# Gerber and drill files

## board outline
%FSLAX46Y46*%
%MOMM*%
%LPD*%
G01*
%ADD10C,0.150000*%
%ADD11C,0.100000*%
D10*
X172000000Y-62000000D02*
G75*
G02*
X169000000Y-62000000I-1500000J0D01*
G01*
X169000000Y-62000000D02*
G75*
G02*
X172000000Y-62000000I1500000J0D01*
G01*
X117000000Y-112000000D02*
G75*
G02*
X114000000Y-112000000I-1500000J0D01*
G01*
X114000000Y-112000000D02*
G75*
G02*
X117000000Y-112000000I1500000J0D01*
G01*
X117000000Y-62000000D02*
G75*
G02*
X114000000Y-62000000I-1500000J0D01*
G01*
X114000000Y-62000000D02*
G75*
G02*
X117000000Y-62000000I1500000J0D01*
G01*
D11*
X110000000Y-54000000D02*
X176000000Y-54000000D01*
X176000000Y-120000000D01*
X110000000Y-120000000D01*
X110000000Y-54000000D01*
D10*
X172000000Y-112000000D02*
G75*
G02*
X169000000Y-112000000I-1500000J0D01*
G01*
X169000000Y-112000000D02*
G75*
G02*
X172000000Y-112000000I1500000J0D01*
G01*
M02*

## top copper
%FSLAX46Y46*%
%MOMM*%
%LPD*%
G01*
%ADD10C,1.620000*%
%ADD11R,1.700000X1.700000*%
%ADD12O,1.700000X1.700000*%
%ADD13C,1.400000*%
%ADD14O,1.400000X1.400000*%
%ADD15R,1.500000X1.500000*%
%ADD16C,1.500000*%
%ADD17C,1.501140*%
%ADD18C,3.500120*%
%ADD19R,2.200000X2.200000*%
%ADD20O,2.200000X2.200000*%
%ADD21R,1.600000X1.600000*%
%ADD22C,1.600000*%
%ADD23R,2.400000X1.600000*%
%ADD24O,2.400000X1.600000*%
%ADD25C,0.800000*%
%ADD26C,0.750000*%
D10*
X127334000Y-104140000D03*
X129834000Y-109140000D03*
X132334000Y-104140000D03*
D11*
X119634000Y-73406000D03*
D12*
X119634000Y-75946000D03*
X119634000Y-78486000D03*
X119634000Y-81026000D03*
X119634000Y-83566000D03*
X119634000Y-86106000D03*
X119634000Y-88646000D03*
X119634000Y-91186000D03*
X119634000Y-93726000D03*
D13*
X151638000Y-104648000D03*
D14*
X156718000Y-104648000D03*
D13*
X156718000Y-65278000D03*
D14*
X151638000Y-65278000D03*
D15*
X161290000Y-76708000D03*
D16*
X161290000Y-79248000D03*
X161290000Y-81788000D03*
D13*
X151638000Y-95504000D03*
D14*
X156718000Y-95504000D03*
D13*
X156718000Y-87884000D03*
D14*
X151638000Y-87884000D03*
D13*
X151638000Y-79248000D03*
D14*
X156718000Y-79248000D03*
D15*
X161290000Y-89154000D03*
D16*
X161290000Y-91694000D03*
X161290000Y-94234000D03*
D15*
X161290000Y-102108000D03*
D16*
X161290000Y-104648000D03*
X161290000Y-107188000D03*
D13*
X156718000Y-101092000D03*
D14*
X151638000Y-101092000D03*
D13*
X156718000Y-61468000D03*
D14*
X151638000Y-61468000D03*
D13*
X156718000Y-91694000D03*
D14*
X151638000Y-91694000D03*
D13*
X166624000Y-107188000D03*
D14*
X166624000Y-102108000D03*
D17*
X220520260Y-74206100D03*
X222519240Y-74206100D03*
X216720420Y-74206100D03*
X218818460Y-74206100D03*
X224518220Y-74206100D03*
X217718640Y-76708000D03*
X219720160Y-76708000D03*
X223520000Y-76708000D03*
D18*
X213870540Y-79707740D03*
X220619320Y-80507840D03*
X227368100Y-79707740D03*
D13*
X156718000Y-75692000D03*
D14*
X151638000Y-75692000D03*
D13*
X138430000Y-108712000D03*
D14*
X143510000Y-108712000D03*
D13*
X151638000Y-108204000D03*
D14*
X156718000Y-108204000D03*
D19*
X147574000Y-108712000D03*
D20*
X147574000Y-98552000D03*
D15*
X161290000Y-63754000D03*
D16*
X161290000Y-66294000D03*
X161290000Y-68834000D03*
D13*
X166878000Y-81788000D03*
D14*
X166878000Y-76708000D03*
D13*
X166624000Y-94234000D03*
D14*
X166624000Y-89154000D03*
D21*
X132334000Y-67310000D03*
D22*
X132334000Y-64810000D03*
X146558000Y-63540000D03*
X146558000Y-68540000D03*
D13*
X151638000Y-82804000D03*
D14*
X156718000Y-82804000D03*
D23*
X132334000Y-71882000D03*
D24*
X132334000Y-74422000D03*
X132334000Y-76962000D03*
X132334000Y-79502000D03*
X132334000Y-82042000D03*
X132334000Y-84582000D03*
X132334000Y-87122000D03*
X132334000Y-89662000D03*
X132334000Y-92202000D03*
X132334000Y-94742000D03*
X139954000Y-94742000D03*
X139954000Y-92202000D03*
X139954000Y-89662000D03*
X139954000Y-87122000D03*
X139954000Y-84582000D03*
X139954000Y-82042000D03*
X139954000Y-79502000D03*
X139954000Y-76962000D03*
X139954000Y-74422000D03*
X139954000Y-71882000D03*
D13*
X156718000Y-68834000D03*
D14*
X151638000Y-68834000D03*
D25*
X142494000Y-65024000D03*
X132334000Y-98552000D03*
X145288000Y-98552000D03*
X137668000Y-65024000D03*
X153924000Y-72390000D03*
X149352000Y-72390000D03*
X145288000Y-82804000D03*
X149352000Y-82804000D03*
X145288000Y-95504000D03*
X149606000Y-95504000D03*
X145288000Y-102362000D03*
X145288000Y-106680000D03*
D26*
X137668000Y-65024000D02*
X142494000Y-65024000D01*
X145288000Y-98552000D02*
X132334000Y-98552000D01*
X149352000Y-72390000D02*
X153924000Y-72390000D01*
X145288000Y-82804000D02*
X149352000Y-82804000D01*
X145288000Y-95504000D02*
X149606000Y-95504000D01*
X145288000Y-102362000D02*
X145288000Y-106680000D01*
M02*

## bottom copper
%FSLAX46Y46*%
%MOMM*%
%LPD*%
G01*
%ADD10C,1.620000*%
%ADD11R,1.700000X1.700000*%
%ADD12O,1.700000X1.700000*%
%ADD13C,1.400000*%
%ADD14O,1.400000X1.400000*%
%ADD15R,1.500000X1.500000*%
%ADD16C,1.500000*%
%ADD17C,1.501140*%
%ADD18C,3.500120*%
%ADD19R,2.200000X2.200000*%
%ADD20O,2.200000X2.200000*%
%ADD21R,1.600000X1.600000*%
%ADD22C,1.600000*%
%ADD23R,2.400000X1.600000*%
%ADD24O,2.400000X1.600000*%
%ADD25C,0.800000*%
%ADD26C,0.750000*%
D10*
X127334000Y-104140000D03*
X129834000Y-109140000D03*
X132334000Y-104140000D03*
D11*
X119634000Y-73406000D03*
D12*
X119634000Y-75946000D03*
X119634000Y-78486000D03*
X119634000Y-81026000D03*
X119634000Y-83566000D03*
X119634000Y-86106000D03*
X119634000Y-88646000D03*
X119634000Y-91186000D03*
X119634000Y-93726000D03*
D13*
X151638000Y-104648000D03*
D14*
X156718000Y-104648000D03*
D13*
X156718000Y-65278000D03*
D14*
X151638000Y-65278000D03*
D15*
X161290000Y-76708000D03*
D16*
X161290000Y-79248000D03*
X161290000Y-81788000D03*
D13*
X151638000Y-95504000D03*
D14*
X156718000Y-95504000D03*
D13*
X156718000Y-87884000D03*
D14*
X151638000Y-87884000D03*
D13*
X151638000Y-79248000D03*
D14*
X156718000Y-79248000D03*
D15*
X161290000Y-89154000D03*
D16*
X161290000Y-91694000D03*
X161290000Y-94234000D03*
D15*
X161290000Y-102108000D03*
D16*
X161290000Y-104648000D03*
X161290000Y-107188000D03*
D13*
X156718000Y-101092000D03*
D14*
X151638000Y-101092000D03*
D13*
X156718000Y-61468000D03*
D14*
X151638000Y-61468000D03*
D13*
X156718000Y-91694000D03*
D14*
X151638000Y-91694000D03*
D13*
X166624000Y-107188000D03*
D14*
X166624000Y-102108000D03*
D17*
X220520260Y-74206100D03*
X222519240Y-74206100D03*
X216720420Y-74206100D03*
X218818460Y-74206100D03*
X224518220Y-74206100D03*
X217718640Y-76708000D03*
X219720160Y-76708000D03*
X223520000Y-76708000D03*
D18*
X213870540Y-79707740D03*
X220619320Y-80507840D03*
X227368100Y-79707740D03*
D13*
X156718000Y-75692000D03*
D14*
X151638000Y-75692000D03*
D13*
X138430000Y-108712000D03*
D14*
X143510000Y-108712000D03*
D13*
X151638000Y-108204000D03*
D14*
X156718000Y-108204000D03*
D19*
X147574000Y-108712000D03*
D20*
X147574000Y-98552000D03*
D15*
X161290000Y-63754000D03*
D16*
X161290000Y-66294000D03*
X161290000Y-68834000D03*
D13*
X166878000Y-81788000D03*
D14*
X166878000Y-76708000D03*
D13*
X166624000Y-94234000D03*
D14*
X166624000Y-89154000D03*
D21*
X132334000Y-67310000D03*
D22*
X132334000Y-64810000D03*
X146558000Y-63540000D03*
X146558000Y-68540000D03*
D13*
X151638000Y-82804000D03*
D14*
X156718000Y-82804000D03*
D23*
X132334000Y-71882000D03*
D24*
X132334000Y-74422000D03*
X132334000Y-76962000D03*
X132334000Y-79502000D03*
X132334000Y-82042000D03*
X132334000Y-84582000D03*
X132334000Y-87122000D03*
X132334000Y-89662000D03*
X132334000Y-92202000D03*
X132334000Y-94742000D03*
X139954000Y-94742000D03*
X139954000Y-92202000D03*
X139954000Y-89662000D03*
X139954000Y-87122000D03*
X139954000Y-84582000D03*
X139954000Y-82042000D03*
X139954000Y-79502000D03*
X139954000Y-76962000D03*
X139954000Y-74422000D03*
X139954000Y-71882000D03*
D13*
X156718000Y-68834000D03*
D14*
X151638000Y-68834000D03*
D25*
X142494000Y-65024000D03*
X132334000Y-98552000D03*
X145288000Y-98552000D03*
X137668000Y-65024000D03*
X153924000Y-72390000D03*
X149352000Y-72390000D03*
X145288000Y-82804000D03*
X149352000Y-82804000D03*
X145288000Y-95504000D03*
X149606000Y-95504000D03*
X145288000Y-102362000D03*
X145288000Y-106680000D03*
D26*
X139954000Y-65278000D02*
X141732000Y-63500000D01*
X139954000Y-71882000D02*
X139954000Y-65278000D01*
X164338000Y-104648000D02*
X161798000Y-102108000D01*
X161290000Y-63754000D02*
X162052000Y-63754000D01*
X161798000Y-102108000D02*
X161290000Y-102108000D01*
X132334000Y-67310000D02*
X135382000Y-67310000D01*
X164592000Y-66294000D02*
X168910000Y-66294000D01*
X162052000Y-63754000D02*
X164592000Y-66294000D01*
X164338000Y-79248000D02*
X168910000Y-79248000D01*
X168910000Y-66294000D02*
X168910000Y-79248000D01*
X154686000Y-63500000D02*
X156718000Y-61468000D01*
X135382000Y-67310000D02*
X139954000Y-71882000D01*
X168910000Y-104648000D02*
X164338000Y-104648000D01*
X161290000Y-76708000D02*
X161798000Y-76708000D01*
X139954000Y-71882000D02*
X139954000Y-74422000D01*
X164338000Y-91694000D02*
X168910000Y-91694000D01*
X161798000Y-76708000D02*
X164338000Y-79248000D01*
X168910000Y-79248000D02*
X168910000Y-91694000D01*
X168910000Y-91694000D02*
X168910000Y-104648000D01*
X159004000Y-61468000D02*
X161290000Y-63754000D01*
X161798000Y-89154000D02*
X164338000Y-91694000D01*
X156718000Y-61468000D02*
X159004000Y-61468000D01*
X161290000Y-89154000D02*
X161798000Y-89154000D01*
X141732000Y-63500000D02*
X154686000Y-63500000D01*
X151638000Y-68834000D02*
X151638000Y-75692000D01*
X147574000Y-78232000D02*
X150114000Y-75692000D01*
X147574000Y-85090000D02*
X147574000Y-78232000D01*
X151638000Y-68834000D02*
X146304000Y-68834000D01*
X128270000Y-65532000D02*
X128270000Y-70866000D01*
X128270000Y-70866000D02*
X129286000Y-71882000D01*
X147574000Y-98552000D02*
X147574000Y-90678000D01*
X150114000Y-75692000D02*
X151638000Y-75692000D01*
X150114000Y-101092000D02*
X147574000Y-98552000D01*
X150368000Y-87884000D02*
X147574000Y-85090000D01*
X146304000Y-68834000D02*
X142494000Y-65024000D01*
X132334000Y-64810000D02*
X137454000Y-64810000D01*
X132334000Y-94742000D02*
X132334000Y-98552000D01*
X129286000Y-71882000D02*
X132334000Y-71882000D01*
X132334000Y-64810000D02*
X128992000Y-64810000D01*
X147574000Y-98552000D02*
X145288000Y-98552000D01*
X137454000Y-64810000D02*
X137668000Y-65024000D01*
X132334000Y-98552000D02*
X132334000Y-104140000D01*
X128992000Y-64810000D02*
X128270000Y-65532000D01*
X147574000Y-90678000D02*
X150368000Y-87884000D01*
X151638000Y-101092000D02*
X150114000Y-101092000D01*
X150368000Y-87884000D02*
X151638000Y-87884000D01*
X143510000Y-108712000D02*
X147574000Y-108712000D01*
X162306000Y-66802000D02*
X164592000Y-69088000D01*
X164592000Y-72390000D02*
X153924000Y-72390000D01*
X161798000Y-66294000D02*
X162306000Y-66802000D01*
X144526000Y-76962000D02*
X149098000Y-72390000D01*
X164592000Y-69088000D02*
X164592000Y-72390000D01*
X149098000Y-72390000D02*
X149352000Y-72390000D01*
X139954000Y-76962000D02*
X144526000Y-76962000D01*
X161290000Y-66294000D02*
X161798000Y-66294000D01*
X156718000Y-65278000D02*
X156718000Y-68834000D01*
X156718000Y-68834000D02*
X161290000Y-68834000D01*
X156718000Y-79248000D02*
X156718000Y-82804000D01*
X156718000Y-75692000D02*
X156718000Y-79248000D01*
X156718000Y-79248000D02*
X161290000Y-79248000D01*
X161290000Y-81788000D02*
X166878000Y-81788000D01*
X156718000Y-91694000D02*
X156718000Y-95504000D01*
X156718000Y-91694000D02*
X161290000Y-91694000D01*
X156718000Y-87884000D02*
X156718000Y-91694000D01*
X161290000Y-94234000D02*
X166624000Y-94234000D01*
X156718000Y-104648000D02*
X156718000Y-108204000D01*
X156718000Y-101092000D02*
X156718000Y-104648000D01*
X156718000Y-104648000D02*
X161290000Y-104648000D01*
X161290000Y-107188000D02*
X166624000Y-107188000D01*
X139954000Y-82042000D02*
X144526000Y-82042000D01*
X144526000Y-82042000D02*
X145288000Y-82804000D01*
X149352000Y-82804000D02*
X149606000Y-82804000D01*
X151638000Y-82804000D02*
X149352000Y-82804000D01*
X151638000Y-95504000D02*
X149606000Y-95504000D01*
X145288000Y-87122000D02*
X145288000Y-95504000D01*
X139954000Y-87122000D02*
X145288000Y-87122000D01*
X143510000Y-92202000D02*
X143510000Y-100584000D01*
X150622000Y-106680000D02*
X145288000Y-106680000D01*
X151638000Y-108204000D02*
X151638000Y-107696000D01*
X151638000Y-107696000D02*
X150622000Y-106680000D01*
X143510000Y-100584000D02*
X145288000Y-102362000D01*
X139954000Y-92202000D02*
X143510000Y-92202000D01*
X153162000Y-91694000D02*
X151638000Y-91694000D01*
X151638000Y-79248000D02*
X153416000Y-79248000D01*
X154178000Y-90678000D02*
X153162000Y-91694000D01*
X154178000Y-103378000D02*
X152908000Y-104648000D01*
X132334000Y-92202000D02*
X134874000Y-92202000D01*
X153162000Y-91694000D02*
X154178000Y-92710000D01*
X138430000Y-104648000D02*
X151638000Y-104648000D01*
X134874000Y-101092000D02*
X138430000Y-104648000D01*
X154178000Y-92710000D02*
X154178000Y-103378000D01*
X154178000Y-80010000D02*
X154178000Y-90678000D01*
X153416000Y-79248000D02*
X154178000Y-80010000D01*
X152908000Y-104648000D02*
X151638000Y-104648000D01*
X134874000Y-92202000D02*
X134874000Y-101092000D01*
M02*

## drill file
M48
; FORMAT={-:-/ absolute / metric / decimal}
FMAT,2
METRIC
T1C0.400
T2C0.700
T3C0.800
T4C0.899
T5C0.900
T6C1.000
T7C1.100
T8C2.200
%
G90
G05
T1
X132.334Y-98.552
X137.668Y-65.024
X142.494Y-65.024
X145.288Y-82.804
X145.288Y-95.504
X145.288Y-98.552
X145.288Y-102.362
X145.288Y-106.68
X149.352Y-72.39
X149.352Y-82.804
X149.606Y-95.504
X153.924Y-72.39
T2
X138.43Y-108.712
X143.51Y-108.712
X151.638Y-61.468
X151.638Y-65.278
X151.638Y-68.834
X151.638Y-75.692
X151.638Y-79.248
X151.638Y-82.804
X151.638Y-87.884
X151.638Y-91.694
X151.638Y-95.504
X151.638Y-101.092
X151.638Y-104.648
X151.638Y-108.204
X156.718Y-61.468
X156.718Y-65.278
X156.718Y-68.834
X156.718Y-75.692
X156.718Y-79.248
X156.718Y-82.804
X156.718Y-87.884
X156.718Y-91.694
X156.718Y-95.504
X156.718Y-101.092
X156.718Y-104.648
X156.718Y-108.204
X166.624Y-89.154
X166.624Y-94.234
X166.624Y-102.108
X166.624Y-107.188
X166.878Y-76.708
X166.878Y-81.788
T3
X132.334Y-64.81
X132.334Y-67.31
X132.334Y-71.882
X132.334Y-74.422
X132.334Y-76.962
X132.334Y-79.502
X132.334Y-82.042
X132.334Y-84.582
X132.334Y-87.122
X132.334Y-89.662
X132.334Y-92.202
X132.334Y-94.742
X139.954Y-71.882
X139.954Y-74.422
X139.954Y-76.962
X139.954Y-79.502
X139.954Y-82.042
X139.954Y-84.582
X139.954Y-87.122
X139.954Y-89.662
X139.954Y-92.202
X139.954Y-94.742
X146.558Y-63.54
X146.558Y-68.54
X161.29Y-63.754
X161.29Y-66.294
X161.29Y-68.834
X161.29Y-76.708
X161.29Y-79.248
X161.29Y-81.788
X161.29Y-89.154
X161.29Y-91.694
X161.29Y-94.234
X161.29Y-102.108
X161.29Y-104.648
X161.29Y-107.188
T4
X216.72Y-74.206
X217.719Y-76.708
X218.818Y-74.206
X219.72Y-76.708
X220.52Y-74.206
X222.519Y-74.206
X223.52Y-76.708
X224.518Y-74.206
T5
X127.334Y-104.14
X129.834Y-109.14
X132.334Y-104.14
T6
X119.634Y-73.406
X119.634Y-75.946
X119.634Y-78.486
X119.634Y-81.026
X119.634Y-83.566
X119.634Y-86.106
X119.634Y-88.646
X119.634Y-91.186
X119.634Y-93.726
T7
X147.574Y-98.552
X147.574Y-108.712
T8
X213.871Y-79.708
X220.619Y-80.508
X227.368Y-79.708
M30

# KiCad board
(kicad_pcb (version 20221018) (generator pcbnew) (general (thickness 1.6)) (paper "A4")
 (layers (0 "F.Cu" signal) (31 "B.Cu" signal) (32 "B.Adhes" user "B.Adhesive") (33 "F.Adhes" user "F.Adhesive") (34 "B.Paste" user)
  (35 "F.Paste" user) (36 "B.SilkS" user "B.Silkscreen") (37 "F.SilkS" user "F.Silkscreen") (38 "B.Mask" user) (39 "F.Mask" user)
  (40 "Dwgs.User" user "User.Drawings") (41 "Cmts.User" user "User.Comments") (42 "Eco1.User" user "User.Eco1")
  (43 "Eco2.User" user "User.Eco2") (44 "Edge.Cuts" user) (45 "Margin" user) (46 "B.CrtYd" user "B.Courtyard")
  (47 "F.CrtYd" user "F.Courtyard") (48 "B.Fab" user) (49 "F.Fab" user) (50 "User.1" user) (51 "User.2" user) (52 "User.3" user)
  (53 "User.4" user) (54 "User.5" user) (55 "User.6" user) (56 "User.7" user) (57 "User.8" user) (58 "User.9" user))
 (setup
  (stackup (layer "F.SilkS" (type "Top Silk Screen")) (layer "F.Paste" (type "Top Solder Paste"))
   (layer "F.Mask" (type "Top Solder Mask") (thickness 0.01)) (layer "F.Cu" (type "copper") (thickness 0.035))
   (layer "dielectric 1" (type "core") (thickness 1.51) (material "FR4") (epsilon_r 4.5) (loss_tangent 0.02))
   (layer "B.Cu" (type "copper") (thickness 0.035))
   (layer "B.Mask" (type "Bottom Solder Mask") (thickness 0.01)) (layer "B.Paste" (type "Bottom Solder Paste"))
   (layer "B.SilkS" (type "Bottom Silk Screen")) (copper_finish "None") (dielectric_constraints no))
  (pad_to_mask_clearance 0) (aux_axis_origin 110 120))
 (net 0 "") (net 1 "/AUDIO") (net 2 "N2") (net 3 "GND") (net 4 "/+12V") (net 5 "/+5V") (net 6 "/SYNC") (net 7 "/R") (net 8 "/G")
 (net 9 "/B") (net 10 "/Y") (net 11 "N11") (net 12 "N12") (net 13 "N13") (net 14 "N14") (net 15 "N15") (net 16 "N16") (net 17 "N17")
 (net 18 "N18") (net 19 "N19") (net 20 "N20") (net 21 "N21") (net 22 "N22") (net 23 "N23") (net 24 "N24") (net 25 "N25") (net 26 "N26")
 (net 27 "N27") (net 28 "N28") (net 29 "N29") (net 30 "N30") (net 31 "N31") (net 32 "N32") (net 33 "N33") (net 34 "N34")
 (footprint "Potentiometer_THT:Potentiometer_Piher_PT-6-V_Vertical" (layer "F.Cu") (at 127.334 104.14 -90)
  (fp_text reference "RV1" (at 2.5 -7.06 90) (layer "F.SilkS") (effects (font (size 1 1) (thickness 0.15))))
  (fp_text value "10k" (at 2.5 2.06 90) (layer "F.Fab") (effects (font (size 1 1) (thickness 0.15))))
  (pad "1" thru_hole circle (at 0 0 270) (size 1.62 1.62) (drill 0.9) (layers "*.Cu" "*.Mask") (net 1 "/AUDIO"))
  (pad "2" thru_hole circle (at 5 -2.5 270) (size 1.62 1.62) (drill 0.9) (layers "*.Cu" "*.Mask") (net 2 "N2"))
  (pad "3" thru_hole circle (at 0 -5 270) (size 1.62 1.62) (drill 0.9) (layers "*.Cu" "*.Mask") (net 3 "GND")))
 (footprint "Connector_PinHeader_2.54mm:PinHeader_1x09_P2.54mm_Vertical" (layer "F.Cu") (at 119.634 73.406)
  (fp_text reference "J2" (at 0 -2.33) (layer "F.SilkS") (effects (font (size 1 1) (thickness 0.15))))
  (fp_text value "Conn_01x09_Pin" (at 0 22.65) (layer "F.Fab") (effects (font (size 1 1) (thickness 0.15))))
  (pad "1" thru_hole rect (at 0 0) (size 1.7 1.7) (drill 1) (layers "*.Cu" "*.Mask") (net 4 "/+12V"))
  (pad "2" thru_hole oval (at 0 2.54) (size 1.7 1.7) (drill 1) (layers "*.Cu" "*.Mask") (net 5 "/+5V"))
  (pad "3" thru_hole oval (at 0 5.08) (size 1.7 1.7) (drill 1) (layers "*.Cu" "*.Mask") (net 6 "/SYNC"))
  (pad "4" thru_hole oval (at 0 7.62) (size 1.7 1.7) (drill 1) (layers "*.Cu" "*.Mask") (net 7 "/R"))
  (pad "5" thru_hole oval (at 0 10.16) (size 1.7 1.7) (drill 1) (layers "*.Cu" "*.Mask") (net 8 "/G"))
  (pad "6" thru_hole oval (at 0 12.7) (size 1.7 1.7) (drill 1) (layers "*.Cu" "*.Mask") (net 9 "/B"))
  (pad "7" thru_hole oval (at 0 15.24) (size 1.7 1.7) (drill 1) (layers "*.Cu" "*.Mask") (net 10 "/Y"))
  (pad "8" thru_hole oval (at 0 17.78) (size 1.7 1.7) (drill 1) (layers "*.Cu" "*.Mask") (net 1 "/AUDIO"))
  (pad "9" thru_hole oval (at 0 20.32) (size 1.7 1.7) (drill 1) (layers "*.Cu" "*.Mask") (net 3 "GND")))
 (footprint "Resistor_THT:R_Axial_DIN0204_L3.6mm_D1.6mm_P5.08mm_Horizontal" (layer "F.Cu") (at 151.638 104.648)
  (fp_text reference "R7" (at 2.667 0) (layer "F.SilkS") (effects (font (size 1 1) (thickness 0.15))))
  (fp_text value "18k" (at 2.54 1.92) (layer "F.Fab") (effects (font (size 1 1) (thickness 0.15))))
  (pad "1" thru_hole circle (at 0 0) (size 1.4 1.4) (drill 0.7) (layers "*.Cu" "*.Mask") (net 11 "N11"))
  (pad "2" thru_hole oval (at 5.08 0) (size 1.4 1.4) (drill 0.7) (layers "*.Cu" "*.Mask") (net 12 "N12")))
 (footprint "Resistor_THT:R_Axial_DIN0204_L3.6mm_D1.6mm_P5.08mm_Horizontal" (layer "F.Cu") (at 156.718 65.278 180)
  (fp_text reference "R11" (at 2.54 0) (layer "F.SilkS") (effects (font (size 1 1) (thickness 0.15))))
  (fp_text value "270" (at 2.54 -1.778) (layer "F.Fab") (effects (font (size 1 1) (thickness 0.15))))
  (pad "1" thru_hole circle (at 0 0 180) (size 1.4 1.4) (drill 0.7) (layers "*.Cu" "*.Mask") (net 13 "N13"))
  (pad "2" thru_hole oval (at 5.08 0 180) (size 1.4 1.4) (drill 0.7) (layers "*.Cu" "*.Mask") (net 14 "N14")))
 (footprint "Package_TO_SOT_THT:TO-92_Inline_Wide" (layer "F.Cu") (at 161.29 76.708 -90)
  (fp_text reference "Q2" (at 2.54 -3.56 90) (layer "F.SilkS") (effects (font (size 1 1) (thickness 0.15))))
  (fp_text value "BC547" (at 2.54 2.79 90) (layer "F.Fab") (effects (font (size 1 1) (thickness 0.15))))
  (pad "1" thru_hole rect (at 0 0 270) (size 1.5 1.5) (drill 0.8) (layers "*.Cu" "*.Mask") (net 5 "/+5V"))
  (pad "2" thru_hole circle (at 2.54 0 270) (size 1.5 1.5) (drill 0.8) (layers "*.Cu" "*.Mask") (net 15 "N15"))
  (pad "3" thru_hole circle (at 5.08 0 270) (size 1.5 1.5) (drill 0.8) (layers "*.Cu" "*.Mask") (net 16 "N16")))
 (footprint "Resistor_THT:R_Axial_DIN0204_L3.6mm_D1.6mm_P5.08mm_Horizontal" (layer "F.Cu") (at 151.638 95.504)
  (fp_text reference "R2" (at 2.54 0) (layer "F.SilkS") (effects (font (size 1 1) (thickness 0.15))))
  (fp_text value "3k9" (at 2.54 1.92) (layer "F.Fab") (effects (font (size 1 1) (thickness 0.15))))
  (pad "1" thru_hole circle (at 0 0) (size 1.4 1.4) (drill 0.7) (layers "*.Cu" "*.Mask") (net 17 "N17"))
  (pad "2" thru_hole oval (at 5.08 0) (size 1.4 1.4) (drill 0.7) (layers "*.Cu" "*.Mask") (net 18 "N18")))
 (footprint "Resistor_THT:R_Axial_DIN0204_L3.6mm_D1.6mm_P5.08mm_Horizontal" (layer "F.Cu") (at 156.718 87.884 180)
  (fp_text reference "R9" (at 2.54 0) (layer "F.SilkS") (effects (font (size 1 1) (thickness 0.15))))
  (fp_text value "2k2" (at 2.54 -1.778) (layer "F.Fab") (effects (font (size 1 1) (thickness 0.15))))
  (pad "1" thru_hole circle (at 0 0 180) (size 1.4 1.4) (drill 0.7) (layers "*.Cu" "*.Mask") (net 18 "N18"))
  (pad "2" thru_hole oval (at 5.08 0 180) (size 1.4 1.4) (drill 0.7) (layers "*.Cu" "*.Mask") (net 3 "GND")))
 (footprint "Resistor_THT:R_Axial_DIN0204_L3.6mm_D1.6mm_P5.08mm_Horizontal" (layer "F.Cu") (at 151.638 79.248)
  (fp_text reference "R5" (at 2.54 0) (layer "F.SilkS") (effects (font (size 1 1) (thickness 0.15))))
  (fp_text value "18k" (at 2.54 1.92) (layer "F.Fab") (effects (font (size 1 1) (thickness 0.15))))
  (pad "1" thru_hole circle (at 0 0) (size 1.4 1.4) (drill 0.7) (layers "*.Cu" "*.Mask") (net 11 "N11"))
  (pad "2" thru_hole oval (at 5.08 0) (size 1.4 1.4) (drill 0.7) (layers "*.Cu" "*.Mask") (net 15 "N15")))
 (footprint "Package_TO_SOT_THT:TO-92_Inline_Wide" (layer "F.Cu") (at 161.29 89.154 -90)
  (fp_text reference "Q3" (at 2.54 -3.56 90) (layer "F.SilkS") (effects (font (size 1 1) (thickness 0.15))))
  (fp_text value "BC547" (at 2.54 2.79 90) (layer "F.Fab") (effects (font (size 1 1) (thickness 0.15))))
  (pad "1" thru_hole rect (at 0 0 270) (size 1.5 1.5) (drill 0.8) (layers "*.Cu" "*.Mask") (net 5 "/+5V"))
  (pad "2" thru_hole circle (at 2.54 0 270) (size 1.5 1.5) (drill 0.8) (layers "*.Cu" "*.Mask") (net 18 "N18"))
  (pad "3" thru_hole circle (at 5.08 0 270) (size 1.5 1.5) (drill 0.8) (layers "*.Cu" "*.Mask") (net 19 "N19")))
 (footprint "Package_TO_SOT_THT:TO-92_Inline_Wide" (layer "F.Cu") (at 161.29 102.108 -90)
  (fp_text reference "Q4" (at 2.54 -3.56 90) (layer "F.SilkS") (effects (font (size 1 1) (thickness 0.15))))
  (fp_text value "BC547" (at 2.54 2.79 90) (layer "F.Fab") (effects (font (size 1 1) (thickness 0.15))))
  (pad "1" thru_hole rect (at 0 0 270) (size 1.5 1.5) (drill 0.8) (layers "*.Cu" "*.Mask") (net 5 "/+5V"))
  (pad "2" thru_hole circle (at 2.54 0 270) (size 1.5 1.5) (drill 0.8) (layers "*.Cu" "*.Mask") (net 12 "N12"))
  (pad "3" thru_hole circle (at 5.08 0 270) (size 1.5 1.5) (drill 0.8) (layers "*.Cu" "*.Mask") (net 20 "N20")))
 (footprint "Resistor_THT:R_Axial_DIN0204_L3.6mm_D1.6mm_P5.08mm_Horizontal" (layer "F.Cu") (at 156.718 101.092 180)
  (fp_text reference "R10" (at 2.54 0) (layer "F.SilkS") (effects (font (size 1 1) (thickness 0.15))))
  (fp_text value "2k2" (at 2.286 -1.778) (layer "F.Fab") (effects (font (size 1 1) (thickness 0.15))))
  (pad "1" thru_hole circle (at 0 0 180) (size 1.4 1.4) (drill 0.7) (layers "*.Cu" "*.Mask") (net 12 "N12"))
  (pad "2" thru_hole oval (at 5.08 0 180) (size 1.4 1.4) (drill 0.7) (layers "*.Cu" "*.Mask") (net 3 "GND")))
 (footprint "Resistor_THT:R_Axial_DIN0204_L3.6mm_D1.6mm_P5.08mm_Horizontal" (layer "F.Cu") (at 156.718 61.468 180)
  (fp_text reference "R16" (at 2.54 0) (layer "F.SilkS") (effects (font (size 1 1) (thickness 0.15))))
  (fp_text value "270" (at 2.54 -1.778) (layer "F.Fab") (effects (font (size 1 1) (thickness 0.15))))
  (pad "1" thru_hole circle (at 0 0 180) (size 1.4 1.4) (drill 0.7) (layers "*.Cu" "*.Mask") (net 5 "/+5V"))
  (pad "2" thru_hole oval (at 5.08 0 180) (size 1.4 1.4) (drill 0.7) (layers "*.Cu" "*.Mask") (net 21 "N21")))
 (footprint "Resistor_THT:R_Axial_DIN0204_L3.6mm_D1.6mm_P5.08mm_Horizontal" (layer "F.Cu") (at 156.718 91.694 180)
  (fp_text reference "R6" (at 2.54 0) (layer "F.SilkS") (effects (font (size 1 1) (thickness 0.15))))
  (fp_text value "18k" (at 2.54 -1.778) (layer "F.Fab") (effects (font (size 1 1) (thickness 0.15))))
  (pad "1" thru_hole circle (at 0 0 180) (size 1.4 1.4) (drill 0.7) (layers "*.Cu" "*.Mask") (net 18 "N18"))
  (pad "2" thru_hole oval (at 5.08 0 180) (size 1.4 1.4) (drill 0.7) (layers "*.Cu" "*.Mask") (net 11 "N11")))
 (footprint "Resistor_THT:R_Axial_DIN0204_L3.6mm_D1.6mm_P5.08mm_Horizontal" (layer "F.Cu") (at 166.624 107.188 90)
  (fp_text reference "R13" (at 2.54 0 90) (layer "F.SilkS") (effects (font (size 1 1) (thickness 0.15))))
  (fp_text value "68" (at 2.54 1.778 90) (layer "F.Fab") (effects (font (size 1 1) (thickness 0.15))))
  (pad "1" thru_hole circle (at 0 0 90) (size 1.4 1.4) (drill 0.7) (layers "*.Cu" "*.Mask") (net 20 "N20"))
  (pad "2" thru_hole oval (at 5.08 0 90) (size 1.4 1.4) (drill 0.7) (layers "*.Cu" "*.Mask") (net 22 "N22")))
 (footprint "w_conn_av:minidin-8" (layer "F.Cu") (at 220.61932 78.70698)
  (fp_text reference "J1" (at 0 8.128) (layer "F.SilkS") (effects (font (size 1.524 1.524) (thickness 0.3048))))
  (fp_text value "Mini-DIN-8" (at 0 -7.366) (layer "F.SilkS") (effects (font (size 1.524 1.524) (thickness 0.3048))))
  (pad "1" thru_hole circle (at -0.09906 -4.50088) (size 1.50114 1.50114) (drill 0.89916) (layers "*.Cu" "*.SilkS" "*.Mask") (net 3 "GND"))
  (pad "2" thru_hole circle (at 1.89992 -4.50088) (size 1.50114 1.50114) (drill 0.89916) (layers "*.Cu" "*.SilkS" "*.Mask") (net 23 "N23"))
  (pad "3" thru_hole circle (at -3.8989 -4.50088) (size 1.50114 1.50114) (drill 0.89916) (layers "*.Cu" "*.SilkS" "*.Mask") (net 21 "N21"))
  (pad "4" thru_hole circle (at -1.80086 -4.50088) (size 1.50114 1.50114) (drill 0.89916) (layers "*.Cu" "*.SilkS" "*.Mask") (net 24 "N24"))
  (pad "5" thru_hole circle (at 3.8989 -4.50088) (size 1.50114 1.50114) (drill 0.89916) (layers "*.Cu" "*.SilkS" "*.Mask") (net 2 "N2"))
  (pad "6" thru_hole circle (at -2.90068 -1.99898) (size 1.50114 1.50114) (drill 0.89916) (layers "*.Cu" "*.SilkS" "*.Mask") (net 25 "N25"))
  (pad "7" thru_hole circle (at -0.89916 -1.99898) (size 1.50114 1.50114) (drill 0.89916) (layers "*.Cu" "*.SilkS" "*.Mask") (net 22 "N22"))
  (pad "8" thru_hole circle (at 2.90068 -1.99898) (size 1.50114 1.50114) (drill 0.89916) (layers "*.Cu" "*.SilkS" "*.Mask") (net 14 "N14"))
  (pad "9" thru_hole circle (at -6.74878 1.00076) (size 3.50012 3.50012) (drill 2.19964) (layers "*.Cu"))
  (pad "10" thru_hole circle (at 0 1.80086) (size 3.50012 3.50012) (drill 2.19964) (layers "*.Cu"))
  (pad "11" thru_hole circle (at 6.74878 1.00076) (size 3.50012 3.50012) (drill 2.19964) (layers "*.Cu")))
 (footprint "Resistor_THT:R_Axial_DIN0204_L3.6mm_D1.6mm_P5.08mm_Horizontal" (layer "F.Cu") (at 156.718 75.692 180)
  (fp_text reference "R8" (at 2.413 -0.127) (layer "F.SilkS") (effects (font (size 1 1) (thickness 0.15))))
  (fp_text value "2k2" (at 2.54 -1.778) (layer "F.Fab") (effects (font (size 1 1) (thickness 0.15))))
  (pad "1" thru_hole circle (at 0 0 180) (size 1.4 1.4) (drill 0.7) (layers "*.Cu" "*.Mask") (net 15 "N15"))
  (pad "2" thru_hole oval (at 5.08 0 180) (size 1.4 1.4) (drill 0.7) (layers "*.Cu" "*.Mask") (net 3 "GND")))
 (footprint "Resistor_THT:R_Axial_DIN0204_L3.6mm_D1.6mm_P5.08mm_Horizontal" (layer "F.Cu") (at 138.43 108.712)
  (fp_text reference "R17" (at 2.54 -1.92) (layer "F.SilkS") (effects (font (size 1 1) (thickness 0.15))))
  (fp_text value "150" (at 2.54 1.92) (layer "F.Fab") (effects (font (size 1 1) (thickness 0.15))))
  (pad "1" thru_hole circle (at 0 0) (size 1.4 1.4) (drill 0.7) (layers "*.Cu" "*.Mask") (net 4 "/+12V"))
  (pad "2" thru_hole oval (at 5.08 0) (size 1.4 1.4) (drill 0.7) (layers "*.Cu" "*.Mask") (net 23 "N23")))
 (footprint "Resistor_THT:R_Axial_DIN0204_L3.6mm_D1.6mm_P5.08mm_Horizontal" (layer "F.Cu") (at 151.638 108.204)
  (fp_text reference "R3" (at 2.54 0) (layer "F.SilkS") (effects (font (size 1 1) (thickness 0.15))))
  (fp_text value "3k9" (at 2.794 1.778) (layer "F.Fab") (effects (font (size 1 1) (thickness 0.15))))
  (pad "1" thru_hole circle (at 0 0) (size 1.4 1.4) (drill 0.7) (layers "*.Cu" "*.Mask") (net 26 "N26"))
  (pad "2" thru_hole oval (at 5.08 0) (size 1.4 1.4) (drill 0.7) (layers "*.Cu" "*.Mask") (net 12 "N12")))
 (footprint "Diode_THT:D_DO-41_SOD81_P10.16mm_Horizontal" (layer "F.Cu") (at 147.574 108.712 90)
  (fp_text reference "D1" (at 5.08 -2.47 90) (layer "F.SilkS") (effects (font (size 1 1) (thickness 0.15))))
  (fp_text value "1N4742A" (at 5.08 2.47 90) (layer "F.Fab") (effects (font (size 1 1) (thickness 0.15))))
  (pad "1" thru_hole rect (at 0 0 90) (size 2.2 2.2) (drill 1.1) (layers "*.Cu" "*.Mask") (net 23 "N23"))
  (pad "2" thru_hole oval (at 10.16 0 90) (size 2.2 2.2) (drill 1.1) (layers "*.Cu" "*.Mask") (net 3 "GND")))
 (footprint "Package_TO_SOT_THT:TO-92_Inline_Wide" (layer "F.Cu") (at 161.29 63.754 -90)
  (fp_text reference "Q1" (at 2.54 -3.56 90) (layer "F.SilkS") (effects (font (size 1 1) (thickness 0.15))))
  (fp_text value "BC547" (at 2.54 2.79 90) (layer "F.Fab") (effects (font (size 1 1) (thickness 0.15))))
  (pad "1" thru_hole rect (at 0 0 270) (size 1.5 1.5) (drill 0.8) (layers "*.Cu" "*.Mask") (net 5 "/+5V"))
  (pad "2" thru_hole circle (at 2.54 0 270) (size 1.5 1.5) (drill 0.8) (layers "*.Cu" "*.Mask") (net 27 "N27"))
  (pad "3" thru_hole circle (at 5.08 0 270) (size 1.5 1.5) (drill 0.8) (layers "*.Cu" "*.Mask") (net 13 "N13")))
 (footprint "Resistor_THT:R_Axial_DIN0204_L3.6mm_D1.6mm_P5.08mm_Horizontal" (layer "F.Cu") (at 166.878 81.788 90)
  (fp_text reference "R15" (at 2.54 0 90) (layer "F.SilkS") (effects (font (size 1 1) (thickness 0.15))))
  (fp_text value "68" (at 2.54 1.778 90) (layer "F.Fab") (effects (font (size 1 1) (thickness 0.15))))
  (pad "1" thru_hole circle (at 0 0 90) (size 1.4 1.4) (drill 0.7) (layers "*.Cu" "*.Mask") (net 16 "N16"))
  (pad "2" thru_hole oval (at 5.08 0 90) (size 1.4 1.4) (drill 0.7) (layers "*.Cu" "*.Mask") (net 25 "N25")))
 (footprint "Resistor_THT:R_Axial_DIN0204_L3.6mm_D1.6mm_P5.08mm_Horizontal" (layer "F.Cu") (at 166.624 94.234 90)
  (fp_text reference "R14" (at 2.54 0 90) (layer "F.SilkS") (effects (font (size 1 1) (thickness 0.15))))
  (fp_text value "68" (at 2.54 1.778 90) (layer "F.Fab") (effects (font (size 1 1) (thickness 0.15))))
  (pad "1" thru_hole circle (at 0 0 90) (size 1.4 1.4) (drill 0.7) (layers "*.Cu" "*.Mask") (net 19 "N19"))
  (pad "2" thru_hole oval (at 5.08 0 90) (size 1.4 1.4) (drill 0.7) (layers "*.Cu" "*.Mask") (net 24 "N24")))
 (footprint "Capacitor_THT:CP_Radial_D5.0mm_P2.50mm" (layer "F.Cu") (at 132.334 67.31 90)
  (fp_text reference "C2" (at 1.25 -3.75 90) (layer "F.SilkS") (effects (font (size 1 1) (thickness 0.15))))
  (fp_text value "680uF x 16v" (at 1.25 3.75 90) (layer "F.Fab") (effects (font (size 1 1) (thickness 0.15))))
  (pad "1" thru_hole rect (at 0 0 90) (size 1.6 1.6) (drill 0.8) (layers "*.Cu" "*.Mask") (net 5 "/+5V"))
  (pad "2" thru_hole circle (at 2.5 0 90) (size 1.6 1.6) (drill 0.8) (layers "*.Cu" "*.Mask") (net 3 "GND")))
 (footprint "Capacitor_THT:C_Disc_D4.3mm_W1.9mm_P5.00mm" (layer "F.Cu") (at 146.558 63.54 -90)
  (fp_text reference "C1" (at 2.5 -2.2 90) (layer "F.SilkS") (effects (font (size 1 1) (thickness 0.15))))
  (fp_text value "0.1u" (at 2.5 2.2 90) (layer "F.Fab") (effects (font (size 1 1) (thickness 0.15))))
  (pad "1" thru_hole circle (at 0 0 270) (size 1.6 1.6) (drill 0.8) (layers "*.Cu" "*.Mask") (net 5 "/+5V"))
  (pad "2" thru_hole circle (at 5 0 270) (size 1.6 1.6) (drill 0.8) (layers "*.Cu" "*.Mask") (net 3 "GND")))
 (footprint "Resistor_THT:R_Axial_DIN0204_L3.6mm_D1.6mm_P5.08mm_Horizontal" (layer "F.Cu") (at 151.638 82.804)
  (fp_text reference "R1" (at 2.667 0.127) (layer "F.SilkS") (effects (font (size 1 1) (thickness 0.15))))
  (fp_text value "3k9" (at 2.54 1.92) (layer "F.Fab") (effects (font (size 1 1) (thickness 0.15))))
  (pad "1" thru_hole circle (at 0 0) (size 1.4 1.4) (drill 0.7) (layers "*.Cu" "*.Mask") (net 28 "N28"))
  (pad "2" thru_hole oval (at 5.08 0) (size 1.4 1.4) (drill 0.7) (layers "*.Cu" "*.Mask") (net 15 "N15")))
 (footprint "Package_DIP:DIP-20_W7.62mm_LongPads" (layer "F.Cu") (at 132.334 71.882)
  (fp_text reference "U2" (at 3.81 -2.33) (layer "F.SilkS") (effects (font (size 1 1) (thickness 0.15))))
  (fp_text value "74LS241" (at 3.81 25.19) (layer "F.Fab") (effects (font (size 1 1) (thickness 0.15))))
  (pad "1" thru_hole rect (at 0 0) (size 2.4 1.6) (drill 0.8) (layers "*.Cu" "*.Mask") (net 3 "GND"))
  (pad "2" thru_hole oval (at 0 2.54) (size 2.4 1.6) (drill 0.8) (layers "*.Cu" "*.Mask") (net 6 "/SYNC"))
  (pad "3" thru_hole oval (at 0 5.08) (size 2.4 1.6) (drill 0.8) (layers "*.Cu" "*.Mask") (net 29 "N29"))
  (pad "4" thru_hole oval (at 0 7.62) (size 2.4 1.6) (drill 0.8) (layers "*.Cu" "*.Mask") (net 7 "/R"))
  (pad "5" thru_hole oval (at 0 10.16) (size 2.4 1.6) (drill 0.8) (layers "*.Cu" "*.Mask") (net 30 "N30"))
  (pad "6" thru_hole oval (at 0 12.7) (size 2.4 1.6) (drill 0.8) (layers "*.Cu" "*.Mask") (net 8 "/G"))
  (pad "7" thru_hole oval (at 0 15.24) (size 2.4 1.6) (drill 0.8) (layers "*.Cu" "*.Mask") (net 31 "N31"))
  (pad "8" thru_hole oval (at 0 17.78) (size 2.4 1.6) (drill 0.8) (layers "*.Cu" "*.Mask") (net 9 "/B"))
  (pad "9" thru_hole oval (at 0 20.32) (size 2.4 1.6) (drill 0.8) (layers "*.Cu" "*.Mask") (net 11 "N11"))
  (pad "10" thru_hole oval (at 0 22.86) (size 2.4 1.6) (drill 0.8) (layers "*.Cu" "*.Mask") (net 3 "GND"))
  (pad "11" thru_hole oval (at 7.62 22.86) (size 2.4 1.6) (drill 0.8) (layers "*.Cu" "*.Mask") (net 10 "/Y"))
  (pad "12" thru_hole oval (at 7.62 20.32) (size 2.4 1.6) (drill 0.8) (layers "*.Cu" "*.Mask") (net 26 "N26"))
  (pad "13" thru_hole oval (at 7.62 17.78) (size 2.4 1.6) (drill 0.8) (layers "*.Cu" "*.Mask") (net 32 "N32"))
  (pad "14" thru_hole oval (at 7.62 15.24) (size 2.4 1.6) (drill 0.8) (layers "*.Cu" "*.Mask") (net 17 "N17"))
  (pad "15" thru_hole oval (at 7.62 12.7) (size 2.4 1.6) (drill 0.8) (layers "*.Cu" "*.Mask") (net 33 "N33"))
  (pad "16" thru_hole oval (at 7.62 10.16) (size 2.4 1.6) (drill 0.8) (layers "*.Cu" "*.Mask") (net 28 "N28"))
  (pad "17" thru_hole oval (at 7.62 7.62) (size 2.4 1.6) (drill 0.8) (layers "*.Cu" "*.Mask") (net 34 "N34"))
  (pad "18" thru_hole oval (at 7.62 5.08) (size 2.4 1.6) (drill 0.8) (layers "*.Cu" "*.Mask") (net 27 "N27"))
  (pad "19" thru_hole oval (at 7.62 2.54) (size 2.4 1.6) (drill 0.8) (layers "*.Cu" "*.Mask") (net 5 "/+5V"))
  (pad "20" thru_hole oval (at 7.62 0) (size 2.4 1.6) (drill 0.8) (layers "*.Cu" "*.Mask") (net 5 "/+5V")))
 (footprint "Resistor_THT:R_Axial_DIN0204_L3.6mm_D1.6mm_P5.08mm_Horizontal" (layer "F.Cu") (at 156.718 68.834 180)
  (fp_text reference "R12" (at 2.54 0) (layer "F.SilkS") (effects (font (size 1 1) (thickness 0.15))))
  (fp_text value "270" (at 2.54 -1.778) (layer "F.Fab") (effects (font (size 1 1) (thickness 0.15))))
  (pad "1" thru_hole circle (at 0 0 180) (size 1.4 1.4) (drill 0.7) (layers "*.Cu" "*.Mask") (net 13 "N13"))
  (pad "2" thru_hole oval (at 5.08 0 180) (size 1.4 1.4) (drill 0.7) (layers "*.Cu" "*.Mask") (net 3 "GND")))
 (gr_circle (center 170.5 62) (end 172 62) (stroke (width 0.15) (type default)) (fill none) (layer "Edge.Cuts"))
 (gr_circle (center 115.5 112) (end 117 112) (stroke (width 0.15) (type default)) (fill none) (layer "Edge.Cuts"))
 (gr_circle (center 115.5 62) (end 117 62) (stroke (width 0.15) (type default)) (fill none) (layer "Edge.Cuts"))
 (gr_rect (start 110 54) (end 176 120) (stroke (width 0.1) (type default)) (fill none) (layer "Edge.Cuts"))
 (gr_circle (center 170.5 112) (end 172 112) (stroke (width 0.15) (type default)) (fill none) (layer "Edge.Cuts"))
 (segment (start 139.954 65.278) (end 141.732 63.5) (width 0.75) (layer "B.Cu") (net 5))
 (segment (start 139.954 71.882) (end 139.954 65.278) (width 0.75) (layer "B.Cu") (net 5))
 (segment (start 164.338 104.648) (end 161.798 102.108) (width 0.75) (layer "B.Cu") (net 5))
 (segment (start 161.29 63.754) (end 162.052 63.754) (width 0.75) (layer "B.Cu") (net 5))
 (segment (start 161.798 102.108) (end 161.29 102.108) (width 0.75) (layer "B.Cu") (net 5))
 (segment (start 132.334 67.31) (end 135.382 67.31) (width 0.75) (layer "B.Cu") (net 5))
 (segment (start 164.592 66.294) (end 168.91 66.294) (width 0.75) (layer "B.Cu") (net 5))
 (segment (start 162.052 63.754) (end 164.592 66.294) (width 0.75) (layer "B.Cu") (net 5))
 (segment (start 164.338 79.248) (end 168.91 79.248) (width 0.75) (layer "B.Cu") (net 5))
 (segment (start 168.91 66.294) (end 168.91 79.248) (width 0.75) (layer "B.Cu") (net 5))
 (segment (start 154.686 63.5) (end 156.718 61.468) (width 0.75) (layer "B.Cu") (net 5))
 (segment (start 135.382 67.31) (end 139.954 71.882) (width 0.75) (layer "B.Cu") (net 5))
 (segment (start 168.91 104.648) (end 164.338 104.648) (width 0.75) (layer "B.Cu") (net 5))
 (segment (start 161.29 76.708) (end 161.798 76.708) (width 0.75) (layer "B.Cu") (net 5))
 (segment (start 139.954 71.882) (end 139.954 74.422) (width 0.75) (layer "B.Cu") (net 5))
 (segment (start 164.338 91.694) (end 168.91 91.694) (width 0.75) (layer "B.Cu") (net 5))
 (segment (start 161.798 76.708) (end 164.338 79.248) (width 0.75) (layer "B.Cu") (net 5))
 (segment (start 168.91 79.248) (end 168.91 91.694) (width 0.75) (layer "B.Cu") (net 5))
 (segment (start 168.91 91.694) (end 168.91 104.648) (width 0.75) (layer "B.Cu") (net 5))
 (segment (start 159.004 61.468) (end 161.29 63.754) (width 0.75) (layer "B.Cu") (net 5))
 (segment (start 161.798 89.154) (end 164.338 91.694) (width 0.75) (layer "B.Cu") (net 5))
 (segment (start 156.718 61.468) (end 159.004 61.468) (width 0.75) (layer "B.Cu") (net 5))
 (segment (start 161.29 89.154) (end 161.798 89.154) (width 0.75) (layer "B.Cu") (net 5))
 (segment (start 141.732 63.5) (end 154.686 63.5) (width 0.75) (layer "B.Cu") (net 5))
 (segment (start 137.668 65.024) (end 142.494 65.024) (width 0.75) (layer "F.Cu") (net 3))
 (segment (start 145.288 98.552) (end 132.334 98.552) (width 0.75) (layer "F.Cu") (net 3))
 (via (at 142.494 65.024) (size 0.8) (drill 0.4) (layers "F.Cu" "B.Cu") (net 3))
 (via (at 132.334 98.552) (size 0.8) (drill 0.4) (layers "F.Cu" "B.Cu") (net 3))
 (via (at 145.288 98.552) (size 0.8) (drill 0.4) (layers "F.Cu" "B.Cu") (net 3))
 (via (at 137.668 65.024) (size 0.8) (drill 0.4) (layers "F.Cu" "B.Cu") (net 3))
 (segment (start 151.638 68.834) (end 151.638 75.692) (width 0.75) (layer "B.Cu") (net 3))
 (segment (start 147.574 78.232) (end 150.114 75.692) (width 0.75) (layer "B.Cu") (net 3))
 (segment (start 147.574 85.09) (end 147.574 78.232) (width 0.75) (layer "B.Cu") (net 3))
 (segment (start 151.638 68.834) (end 146.304 68.834) (width 0.75) (layer "B.Cu") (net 3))
 (segment (start 128.27 65.532) (end 128.27 70.866) (width 0.75) (layer "B.Cu") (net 3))
 (segment (start 128.27 70.866) (end 129.286 71.882) (width 0.75) (layer "B.Cu") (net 3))
 (segment (start 147.574 98.552) (end 147.574 90.678) (width 0.75) (layer "B.Cu") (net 3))
 (segment (start 150.114 75.692) (end 151.638 75.692) (width 0.75) (layer "B.Cu") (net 3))
 (segment (start 150.114 101.092) (end 147.574 98.552) (width 0.75) (layer "B.Cu") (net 3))
 (segment (start 150.368 87.884) (end 147.574 85.09) (width 0.75) (layer "B.Cu") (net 3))
 (segment (start 146.304 68.834) (end 142.494 65.024) (width 0.75) (layer "B.Cu") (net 3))
 (segment (start 132.334 64.81) (end 137.454 64.81) (width 0.75) (layer "B.Cu") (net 3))
 (segment (start 132.334 94.742) (end 132.334 98.552) (width 0.75) (layer "B.Cu") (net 3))
 (segment (start 129.286 71.882) (end 132.334 71.882) (width 0.75) (layer "B.Cu") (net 3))
 (segment (start 132.334 64.81) (end 128.992 64.81) (width 0.75) (layer "B.Cu") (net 3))
 (segment (start 147.574 98.552) (end 145.288 98.552) (width 0.75) (layer "B.Cu") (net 3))
 (segment (start 137.454 64.81) (end 137.668 65.024) (width 0.75) (layer "B.Cu") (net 3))
 (segment (start 132.334 98.552) (end 132.334 104.14) (width 0.75) (layer "B.Cu") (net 3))
 (segment (start 128.992 64.81) (end 128.27 65.532) (width 0.75) (layer "B.Cu") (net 3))
 (segment (start 147.574 90.678) (end 150.368 87.884) (width 0.75) (layer "B.Cu") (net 3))
 (segment (start 151.638 101.092) (end 150.114 101.092) (width 0.75) (layer "B.Cu") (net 3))
 (segment (start 150.368 87.884) (end 151.638 87.884) (width 0.75) (layer "B.Cu") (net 3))
 (segment (start 143.51 108.712) (end 147.574 108.712) (width 0.75) (layer "B.Cu") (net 23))
 (segment (start 149.352 72.39) (end 153.924 72.39) (width 0.75) (layer "F.Cu") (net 27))
 (via (at 153.924 72.39) (size 0.8) (drill 0.4) (layers "F.Cu" "B.Cu") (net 27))
 (via (at 149.352 72.39) (size 0.8) (drill 0.4) (layers "F.Cu" "B.Cu") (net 27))
 (segment (start 162.306 66.802) (end 164.592 69.088) (width 0.75) (layer "B.Cu") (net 27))
 (segment (start 164.592 72.39) (end 153.924 72.39) (width 0.75) (layer "B.Cu") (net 27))
 (segment (start 161.798 66.294) (end 162.306 66.802) (width 0.75) (layer "B.Cu") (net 27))
 (segment (start 144.526 76.962) (end 149.098 72.39) (width 0.75) (layer "B.Cu") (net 27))
 (segment (start 164.592 69.088) (end 164.592 72.39) (width 0.75) (layer "B.Cu") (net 27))
 (segment (start 149.098 72.39) (end 149.352 72.39) (width 0.75) (layer "B.Cu") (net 27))
 (segment (start 139.954 76.962) (end 144.526 76.962) (width 0.75) (layer "B.Cu") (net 27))
 (segment (start 161.29 66.294) (end 161.798 66.294) (width 0.75) (layer "B.Cu") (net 27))
 (segment (start 156.718 65.278) (end 156.718 68.834) (width 0.75) (layer "B.Cu") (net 13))
 (segment (start 156.718 68.834) (end 161.29 68.834) (width 0.75) (layer "B.Cu") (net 13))
 (segment (start 156.718 79.248) (end 156.718 82.804) (width 0.75) (layer "B.Cu") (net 15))
 (segment (start 156.718 75.692) (end 156.718 79.248) (width 0.75) (layer "B.Cu") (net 15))
 (segment (start 156.718 79.248) (end 161.29 79.248) (width 0.75) (layer "B.Cu") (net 15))
 (segment (start 161.29 81.788) (end 166.878 81.788) (width 0.75) (layer "B.Cu") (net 16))
 (segment (start 156.718 91.694) (end 156.718 95.504) (width 0.75) (layer "B.Cu") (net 18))
 (segment (start 156.718 91.694) (end 161.29 91.694) (width 0.75) (layer "B.Cu") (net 18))
 (segment (start 156.718 87.884) (end 156.718 91.694) (width 0.75) (layer "B.Cu") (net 18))
 (segment (start 161.29 94.234) (end 166.624 94.234) (width 0.75) (layer "B.Cu") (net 19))
 (segment (start 156.718 104.648) (end 156.718 108.204) (width 0.75) (layer "B.Cu") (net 12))
 (segment (start 156.718 101.092) (end 156.718 104.648) (width 0.75) (layer "B.Cu") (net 12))
 (segment (start 156.718 104.648) (end 161.29 104.648) (width 0.75) (layer "B.Cu") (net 12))
 (segment (start 161.29 107.188) (end 166.624 107.188) (width 0.75) (layer "B.Cu") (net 20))
 (segment (start 145.288 82.804) (end 149.352 82.804) (width 0.75) (layer "F.Cu") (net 28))
 (via (at 145.288 82.804) (size 0.8) (drill 0.4) (layers "F.Cu" "B.Cu") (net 28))
 (via (at 149.352 82.804) (size 0.8) (drill 0.4) (layers "F.Cu" "B.Cu") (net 28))
 (segment (start 139.954 82.042) (end 144.526 82.042) (width 0.75) (layer "B.Cu") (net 28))
 (segment (start 144.526 82.042) (end 145.288 82.804) (width 0.75) (layer "B.Cu") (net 28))
 (segment (start 149.352 82.804) (end 149.606 82.804) (width 0.75) (layer "B.Cu") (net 28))
 (segment (start 151.638 82.804) (end 149.352 82.804) (width 0.75) (layer "B.Cu") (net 28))
 (segment (start 145.288 95.504) (end 149.606 95.504) (width 0.75) (layer "F.Cu") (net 17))
 (via (at 145.288 95.504) (size 0.8) (drill 0.4) (layers "F.Cu" "B.Cu") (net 17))
 (via (at 149.606 95.504) (size 0.8) (drill 0.4) (layers "F.Cu" "B.Cu") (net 17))
 (segment (start 151.638 95.504) (end 149.606 95.504) (width 0.75) (layer "B.Cu") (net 17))
 (segment (start 145.288 87.122) (end 145.288 95.504) (width 0.75) (layer "B.Cu") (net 17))
 (segment (start 139.954 87.122) (end 145.288 87.122) (width 0.75) (layer "B.Cu") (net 17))
 (segment (start 145.288 102.362) (end 145.288 106.68) (width 0.75) (layer "F.Cu") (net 26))
 (via (at 145.288 102.362) (size 0.8) (drill 0.4) (layers "F.Cu" "B.Cu") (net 26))
 (via (at 145.288 106.68) (size 0.8) (drill 0.4) (layers "F.Cu" "B.Cu") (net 26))
 (segment (start 143.51 92.202) (end 143.51 100.584) (width 0.75) (layer "B.Cu") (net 26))
 (segment (start 150.622 106.68) (end 145.288 106.68) (width 0.75) (layer "B.Cu") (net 26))
 (segment (start 151.638 108.204) (end 151.638 107.696) (width 0.75) (layer "B.Cu") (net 26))
 (segment (start 151.638 107.696) (end 150.622 106.68) (width 0.75) (layer "B.Cu") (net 26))
 (segment (start 143.51 100.584) (end 145.288 102.362) (width 0.75) (layer "B.Cu") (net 26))
 (segment (start 139.954 92.202) (end 143.51 92.202) (width 0.75) (layer "B.Cu") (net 26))
 (segment (start 153.162 91.694) (end 151.638 91.694) (width 0.75) (layer "B.Cu") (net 11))
 (segment (start 151.638 79.248) (end 153.416 79.248) (width 0.75) (layer "B.Cu") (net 11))
 (segment (start 154.178 90.678) (end 153.162 91.694) (width 0.75) (layer "B.Cu") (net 11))
 (segment (start 154.178 103.378) (end 152.908 104.648) (width 0.75) (layer "B.Cu") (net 11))
 (segment (start 132.334 92.202) (end 134.874 92.202) (width 0.75) (layer "B.Cu") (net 11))
 (segment (start 153.162 91.694) (end 154.178 92.71) (width 0.75) (layer "B.Cu") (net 11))
 (segment (start 138.43 104.648) (end 151.638 104.648) (width 0.75) (layer "B.Cu") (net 11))
 (segment (start 134.874 101.092) (end 138.43 104.648) (width 0.75) (layer "B.Cu") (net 11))
 (segment (start 154.178 92.71) (end 154.178 103.378) (width 0.75) (layer "B.Cu") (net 11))
 (segment (start 154.178 80.01) (end 154.178 90.678) (width 0.75) (layer "B.Cu") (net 11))
 (segment (start 153.416 79.248) (end 154.178 80.01) (width 0.75) (layer "B.Cu") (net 11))
 (segment (start 152.908 104.648) (end 151.638 104.648) (width 0.75) (layer "B.Cu") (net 11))
 (segment (start 134.874 92.202) (end 134.874 101.092) (width 0.75) (layer "B.Cu") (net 11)))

